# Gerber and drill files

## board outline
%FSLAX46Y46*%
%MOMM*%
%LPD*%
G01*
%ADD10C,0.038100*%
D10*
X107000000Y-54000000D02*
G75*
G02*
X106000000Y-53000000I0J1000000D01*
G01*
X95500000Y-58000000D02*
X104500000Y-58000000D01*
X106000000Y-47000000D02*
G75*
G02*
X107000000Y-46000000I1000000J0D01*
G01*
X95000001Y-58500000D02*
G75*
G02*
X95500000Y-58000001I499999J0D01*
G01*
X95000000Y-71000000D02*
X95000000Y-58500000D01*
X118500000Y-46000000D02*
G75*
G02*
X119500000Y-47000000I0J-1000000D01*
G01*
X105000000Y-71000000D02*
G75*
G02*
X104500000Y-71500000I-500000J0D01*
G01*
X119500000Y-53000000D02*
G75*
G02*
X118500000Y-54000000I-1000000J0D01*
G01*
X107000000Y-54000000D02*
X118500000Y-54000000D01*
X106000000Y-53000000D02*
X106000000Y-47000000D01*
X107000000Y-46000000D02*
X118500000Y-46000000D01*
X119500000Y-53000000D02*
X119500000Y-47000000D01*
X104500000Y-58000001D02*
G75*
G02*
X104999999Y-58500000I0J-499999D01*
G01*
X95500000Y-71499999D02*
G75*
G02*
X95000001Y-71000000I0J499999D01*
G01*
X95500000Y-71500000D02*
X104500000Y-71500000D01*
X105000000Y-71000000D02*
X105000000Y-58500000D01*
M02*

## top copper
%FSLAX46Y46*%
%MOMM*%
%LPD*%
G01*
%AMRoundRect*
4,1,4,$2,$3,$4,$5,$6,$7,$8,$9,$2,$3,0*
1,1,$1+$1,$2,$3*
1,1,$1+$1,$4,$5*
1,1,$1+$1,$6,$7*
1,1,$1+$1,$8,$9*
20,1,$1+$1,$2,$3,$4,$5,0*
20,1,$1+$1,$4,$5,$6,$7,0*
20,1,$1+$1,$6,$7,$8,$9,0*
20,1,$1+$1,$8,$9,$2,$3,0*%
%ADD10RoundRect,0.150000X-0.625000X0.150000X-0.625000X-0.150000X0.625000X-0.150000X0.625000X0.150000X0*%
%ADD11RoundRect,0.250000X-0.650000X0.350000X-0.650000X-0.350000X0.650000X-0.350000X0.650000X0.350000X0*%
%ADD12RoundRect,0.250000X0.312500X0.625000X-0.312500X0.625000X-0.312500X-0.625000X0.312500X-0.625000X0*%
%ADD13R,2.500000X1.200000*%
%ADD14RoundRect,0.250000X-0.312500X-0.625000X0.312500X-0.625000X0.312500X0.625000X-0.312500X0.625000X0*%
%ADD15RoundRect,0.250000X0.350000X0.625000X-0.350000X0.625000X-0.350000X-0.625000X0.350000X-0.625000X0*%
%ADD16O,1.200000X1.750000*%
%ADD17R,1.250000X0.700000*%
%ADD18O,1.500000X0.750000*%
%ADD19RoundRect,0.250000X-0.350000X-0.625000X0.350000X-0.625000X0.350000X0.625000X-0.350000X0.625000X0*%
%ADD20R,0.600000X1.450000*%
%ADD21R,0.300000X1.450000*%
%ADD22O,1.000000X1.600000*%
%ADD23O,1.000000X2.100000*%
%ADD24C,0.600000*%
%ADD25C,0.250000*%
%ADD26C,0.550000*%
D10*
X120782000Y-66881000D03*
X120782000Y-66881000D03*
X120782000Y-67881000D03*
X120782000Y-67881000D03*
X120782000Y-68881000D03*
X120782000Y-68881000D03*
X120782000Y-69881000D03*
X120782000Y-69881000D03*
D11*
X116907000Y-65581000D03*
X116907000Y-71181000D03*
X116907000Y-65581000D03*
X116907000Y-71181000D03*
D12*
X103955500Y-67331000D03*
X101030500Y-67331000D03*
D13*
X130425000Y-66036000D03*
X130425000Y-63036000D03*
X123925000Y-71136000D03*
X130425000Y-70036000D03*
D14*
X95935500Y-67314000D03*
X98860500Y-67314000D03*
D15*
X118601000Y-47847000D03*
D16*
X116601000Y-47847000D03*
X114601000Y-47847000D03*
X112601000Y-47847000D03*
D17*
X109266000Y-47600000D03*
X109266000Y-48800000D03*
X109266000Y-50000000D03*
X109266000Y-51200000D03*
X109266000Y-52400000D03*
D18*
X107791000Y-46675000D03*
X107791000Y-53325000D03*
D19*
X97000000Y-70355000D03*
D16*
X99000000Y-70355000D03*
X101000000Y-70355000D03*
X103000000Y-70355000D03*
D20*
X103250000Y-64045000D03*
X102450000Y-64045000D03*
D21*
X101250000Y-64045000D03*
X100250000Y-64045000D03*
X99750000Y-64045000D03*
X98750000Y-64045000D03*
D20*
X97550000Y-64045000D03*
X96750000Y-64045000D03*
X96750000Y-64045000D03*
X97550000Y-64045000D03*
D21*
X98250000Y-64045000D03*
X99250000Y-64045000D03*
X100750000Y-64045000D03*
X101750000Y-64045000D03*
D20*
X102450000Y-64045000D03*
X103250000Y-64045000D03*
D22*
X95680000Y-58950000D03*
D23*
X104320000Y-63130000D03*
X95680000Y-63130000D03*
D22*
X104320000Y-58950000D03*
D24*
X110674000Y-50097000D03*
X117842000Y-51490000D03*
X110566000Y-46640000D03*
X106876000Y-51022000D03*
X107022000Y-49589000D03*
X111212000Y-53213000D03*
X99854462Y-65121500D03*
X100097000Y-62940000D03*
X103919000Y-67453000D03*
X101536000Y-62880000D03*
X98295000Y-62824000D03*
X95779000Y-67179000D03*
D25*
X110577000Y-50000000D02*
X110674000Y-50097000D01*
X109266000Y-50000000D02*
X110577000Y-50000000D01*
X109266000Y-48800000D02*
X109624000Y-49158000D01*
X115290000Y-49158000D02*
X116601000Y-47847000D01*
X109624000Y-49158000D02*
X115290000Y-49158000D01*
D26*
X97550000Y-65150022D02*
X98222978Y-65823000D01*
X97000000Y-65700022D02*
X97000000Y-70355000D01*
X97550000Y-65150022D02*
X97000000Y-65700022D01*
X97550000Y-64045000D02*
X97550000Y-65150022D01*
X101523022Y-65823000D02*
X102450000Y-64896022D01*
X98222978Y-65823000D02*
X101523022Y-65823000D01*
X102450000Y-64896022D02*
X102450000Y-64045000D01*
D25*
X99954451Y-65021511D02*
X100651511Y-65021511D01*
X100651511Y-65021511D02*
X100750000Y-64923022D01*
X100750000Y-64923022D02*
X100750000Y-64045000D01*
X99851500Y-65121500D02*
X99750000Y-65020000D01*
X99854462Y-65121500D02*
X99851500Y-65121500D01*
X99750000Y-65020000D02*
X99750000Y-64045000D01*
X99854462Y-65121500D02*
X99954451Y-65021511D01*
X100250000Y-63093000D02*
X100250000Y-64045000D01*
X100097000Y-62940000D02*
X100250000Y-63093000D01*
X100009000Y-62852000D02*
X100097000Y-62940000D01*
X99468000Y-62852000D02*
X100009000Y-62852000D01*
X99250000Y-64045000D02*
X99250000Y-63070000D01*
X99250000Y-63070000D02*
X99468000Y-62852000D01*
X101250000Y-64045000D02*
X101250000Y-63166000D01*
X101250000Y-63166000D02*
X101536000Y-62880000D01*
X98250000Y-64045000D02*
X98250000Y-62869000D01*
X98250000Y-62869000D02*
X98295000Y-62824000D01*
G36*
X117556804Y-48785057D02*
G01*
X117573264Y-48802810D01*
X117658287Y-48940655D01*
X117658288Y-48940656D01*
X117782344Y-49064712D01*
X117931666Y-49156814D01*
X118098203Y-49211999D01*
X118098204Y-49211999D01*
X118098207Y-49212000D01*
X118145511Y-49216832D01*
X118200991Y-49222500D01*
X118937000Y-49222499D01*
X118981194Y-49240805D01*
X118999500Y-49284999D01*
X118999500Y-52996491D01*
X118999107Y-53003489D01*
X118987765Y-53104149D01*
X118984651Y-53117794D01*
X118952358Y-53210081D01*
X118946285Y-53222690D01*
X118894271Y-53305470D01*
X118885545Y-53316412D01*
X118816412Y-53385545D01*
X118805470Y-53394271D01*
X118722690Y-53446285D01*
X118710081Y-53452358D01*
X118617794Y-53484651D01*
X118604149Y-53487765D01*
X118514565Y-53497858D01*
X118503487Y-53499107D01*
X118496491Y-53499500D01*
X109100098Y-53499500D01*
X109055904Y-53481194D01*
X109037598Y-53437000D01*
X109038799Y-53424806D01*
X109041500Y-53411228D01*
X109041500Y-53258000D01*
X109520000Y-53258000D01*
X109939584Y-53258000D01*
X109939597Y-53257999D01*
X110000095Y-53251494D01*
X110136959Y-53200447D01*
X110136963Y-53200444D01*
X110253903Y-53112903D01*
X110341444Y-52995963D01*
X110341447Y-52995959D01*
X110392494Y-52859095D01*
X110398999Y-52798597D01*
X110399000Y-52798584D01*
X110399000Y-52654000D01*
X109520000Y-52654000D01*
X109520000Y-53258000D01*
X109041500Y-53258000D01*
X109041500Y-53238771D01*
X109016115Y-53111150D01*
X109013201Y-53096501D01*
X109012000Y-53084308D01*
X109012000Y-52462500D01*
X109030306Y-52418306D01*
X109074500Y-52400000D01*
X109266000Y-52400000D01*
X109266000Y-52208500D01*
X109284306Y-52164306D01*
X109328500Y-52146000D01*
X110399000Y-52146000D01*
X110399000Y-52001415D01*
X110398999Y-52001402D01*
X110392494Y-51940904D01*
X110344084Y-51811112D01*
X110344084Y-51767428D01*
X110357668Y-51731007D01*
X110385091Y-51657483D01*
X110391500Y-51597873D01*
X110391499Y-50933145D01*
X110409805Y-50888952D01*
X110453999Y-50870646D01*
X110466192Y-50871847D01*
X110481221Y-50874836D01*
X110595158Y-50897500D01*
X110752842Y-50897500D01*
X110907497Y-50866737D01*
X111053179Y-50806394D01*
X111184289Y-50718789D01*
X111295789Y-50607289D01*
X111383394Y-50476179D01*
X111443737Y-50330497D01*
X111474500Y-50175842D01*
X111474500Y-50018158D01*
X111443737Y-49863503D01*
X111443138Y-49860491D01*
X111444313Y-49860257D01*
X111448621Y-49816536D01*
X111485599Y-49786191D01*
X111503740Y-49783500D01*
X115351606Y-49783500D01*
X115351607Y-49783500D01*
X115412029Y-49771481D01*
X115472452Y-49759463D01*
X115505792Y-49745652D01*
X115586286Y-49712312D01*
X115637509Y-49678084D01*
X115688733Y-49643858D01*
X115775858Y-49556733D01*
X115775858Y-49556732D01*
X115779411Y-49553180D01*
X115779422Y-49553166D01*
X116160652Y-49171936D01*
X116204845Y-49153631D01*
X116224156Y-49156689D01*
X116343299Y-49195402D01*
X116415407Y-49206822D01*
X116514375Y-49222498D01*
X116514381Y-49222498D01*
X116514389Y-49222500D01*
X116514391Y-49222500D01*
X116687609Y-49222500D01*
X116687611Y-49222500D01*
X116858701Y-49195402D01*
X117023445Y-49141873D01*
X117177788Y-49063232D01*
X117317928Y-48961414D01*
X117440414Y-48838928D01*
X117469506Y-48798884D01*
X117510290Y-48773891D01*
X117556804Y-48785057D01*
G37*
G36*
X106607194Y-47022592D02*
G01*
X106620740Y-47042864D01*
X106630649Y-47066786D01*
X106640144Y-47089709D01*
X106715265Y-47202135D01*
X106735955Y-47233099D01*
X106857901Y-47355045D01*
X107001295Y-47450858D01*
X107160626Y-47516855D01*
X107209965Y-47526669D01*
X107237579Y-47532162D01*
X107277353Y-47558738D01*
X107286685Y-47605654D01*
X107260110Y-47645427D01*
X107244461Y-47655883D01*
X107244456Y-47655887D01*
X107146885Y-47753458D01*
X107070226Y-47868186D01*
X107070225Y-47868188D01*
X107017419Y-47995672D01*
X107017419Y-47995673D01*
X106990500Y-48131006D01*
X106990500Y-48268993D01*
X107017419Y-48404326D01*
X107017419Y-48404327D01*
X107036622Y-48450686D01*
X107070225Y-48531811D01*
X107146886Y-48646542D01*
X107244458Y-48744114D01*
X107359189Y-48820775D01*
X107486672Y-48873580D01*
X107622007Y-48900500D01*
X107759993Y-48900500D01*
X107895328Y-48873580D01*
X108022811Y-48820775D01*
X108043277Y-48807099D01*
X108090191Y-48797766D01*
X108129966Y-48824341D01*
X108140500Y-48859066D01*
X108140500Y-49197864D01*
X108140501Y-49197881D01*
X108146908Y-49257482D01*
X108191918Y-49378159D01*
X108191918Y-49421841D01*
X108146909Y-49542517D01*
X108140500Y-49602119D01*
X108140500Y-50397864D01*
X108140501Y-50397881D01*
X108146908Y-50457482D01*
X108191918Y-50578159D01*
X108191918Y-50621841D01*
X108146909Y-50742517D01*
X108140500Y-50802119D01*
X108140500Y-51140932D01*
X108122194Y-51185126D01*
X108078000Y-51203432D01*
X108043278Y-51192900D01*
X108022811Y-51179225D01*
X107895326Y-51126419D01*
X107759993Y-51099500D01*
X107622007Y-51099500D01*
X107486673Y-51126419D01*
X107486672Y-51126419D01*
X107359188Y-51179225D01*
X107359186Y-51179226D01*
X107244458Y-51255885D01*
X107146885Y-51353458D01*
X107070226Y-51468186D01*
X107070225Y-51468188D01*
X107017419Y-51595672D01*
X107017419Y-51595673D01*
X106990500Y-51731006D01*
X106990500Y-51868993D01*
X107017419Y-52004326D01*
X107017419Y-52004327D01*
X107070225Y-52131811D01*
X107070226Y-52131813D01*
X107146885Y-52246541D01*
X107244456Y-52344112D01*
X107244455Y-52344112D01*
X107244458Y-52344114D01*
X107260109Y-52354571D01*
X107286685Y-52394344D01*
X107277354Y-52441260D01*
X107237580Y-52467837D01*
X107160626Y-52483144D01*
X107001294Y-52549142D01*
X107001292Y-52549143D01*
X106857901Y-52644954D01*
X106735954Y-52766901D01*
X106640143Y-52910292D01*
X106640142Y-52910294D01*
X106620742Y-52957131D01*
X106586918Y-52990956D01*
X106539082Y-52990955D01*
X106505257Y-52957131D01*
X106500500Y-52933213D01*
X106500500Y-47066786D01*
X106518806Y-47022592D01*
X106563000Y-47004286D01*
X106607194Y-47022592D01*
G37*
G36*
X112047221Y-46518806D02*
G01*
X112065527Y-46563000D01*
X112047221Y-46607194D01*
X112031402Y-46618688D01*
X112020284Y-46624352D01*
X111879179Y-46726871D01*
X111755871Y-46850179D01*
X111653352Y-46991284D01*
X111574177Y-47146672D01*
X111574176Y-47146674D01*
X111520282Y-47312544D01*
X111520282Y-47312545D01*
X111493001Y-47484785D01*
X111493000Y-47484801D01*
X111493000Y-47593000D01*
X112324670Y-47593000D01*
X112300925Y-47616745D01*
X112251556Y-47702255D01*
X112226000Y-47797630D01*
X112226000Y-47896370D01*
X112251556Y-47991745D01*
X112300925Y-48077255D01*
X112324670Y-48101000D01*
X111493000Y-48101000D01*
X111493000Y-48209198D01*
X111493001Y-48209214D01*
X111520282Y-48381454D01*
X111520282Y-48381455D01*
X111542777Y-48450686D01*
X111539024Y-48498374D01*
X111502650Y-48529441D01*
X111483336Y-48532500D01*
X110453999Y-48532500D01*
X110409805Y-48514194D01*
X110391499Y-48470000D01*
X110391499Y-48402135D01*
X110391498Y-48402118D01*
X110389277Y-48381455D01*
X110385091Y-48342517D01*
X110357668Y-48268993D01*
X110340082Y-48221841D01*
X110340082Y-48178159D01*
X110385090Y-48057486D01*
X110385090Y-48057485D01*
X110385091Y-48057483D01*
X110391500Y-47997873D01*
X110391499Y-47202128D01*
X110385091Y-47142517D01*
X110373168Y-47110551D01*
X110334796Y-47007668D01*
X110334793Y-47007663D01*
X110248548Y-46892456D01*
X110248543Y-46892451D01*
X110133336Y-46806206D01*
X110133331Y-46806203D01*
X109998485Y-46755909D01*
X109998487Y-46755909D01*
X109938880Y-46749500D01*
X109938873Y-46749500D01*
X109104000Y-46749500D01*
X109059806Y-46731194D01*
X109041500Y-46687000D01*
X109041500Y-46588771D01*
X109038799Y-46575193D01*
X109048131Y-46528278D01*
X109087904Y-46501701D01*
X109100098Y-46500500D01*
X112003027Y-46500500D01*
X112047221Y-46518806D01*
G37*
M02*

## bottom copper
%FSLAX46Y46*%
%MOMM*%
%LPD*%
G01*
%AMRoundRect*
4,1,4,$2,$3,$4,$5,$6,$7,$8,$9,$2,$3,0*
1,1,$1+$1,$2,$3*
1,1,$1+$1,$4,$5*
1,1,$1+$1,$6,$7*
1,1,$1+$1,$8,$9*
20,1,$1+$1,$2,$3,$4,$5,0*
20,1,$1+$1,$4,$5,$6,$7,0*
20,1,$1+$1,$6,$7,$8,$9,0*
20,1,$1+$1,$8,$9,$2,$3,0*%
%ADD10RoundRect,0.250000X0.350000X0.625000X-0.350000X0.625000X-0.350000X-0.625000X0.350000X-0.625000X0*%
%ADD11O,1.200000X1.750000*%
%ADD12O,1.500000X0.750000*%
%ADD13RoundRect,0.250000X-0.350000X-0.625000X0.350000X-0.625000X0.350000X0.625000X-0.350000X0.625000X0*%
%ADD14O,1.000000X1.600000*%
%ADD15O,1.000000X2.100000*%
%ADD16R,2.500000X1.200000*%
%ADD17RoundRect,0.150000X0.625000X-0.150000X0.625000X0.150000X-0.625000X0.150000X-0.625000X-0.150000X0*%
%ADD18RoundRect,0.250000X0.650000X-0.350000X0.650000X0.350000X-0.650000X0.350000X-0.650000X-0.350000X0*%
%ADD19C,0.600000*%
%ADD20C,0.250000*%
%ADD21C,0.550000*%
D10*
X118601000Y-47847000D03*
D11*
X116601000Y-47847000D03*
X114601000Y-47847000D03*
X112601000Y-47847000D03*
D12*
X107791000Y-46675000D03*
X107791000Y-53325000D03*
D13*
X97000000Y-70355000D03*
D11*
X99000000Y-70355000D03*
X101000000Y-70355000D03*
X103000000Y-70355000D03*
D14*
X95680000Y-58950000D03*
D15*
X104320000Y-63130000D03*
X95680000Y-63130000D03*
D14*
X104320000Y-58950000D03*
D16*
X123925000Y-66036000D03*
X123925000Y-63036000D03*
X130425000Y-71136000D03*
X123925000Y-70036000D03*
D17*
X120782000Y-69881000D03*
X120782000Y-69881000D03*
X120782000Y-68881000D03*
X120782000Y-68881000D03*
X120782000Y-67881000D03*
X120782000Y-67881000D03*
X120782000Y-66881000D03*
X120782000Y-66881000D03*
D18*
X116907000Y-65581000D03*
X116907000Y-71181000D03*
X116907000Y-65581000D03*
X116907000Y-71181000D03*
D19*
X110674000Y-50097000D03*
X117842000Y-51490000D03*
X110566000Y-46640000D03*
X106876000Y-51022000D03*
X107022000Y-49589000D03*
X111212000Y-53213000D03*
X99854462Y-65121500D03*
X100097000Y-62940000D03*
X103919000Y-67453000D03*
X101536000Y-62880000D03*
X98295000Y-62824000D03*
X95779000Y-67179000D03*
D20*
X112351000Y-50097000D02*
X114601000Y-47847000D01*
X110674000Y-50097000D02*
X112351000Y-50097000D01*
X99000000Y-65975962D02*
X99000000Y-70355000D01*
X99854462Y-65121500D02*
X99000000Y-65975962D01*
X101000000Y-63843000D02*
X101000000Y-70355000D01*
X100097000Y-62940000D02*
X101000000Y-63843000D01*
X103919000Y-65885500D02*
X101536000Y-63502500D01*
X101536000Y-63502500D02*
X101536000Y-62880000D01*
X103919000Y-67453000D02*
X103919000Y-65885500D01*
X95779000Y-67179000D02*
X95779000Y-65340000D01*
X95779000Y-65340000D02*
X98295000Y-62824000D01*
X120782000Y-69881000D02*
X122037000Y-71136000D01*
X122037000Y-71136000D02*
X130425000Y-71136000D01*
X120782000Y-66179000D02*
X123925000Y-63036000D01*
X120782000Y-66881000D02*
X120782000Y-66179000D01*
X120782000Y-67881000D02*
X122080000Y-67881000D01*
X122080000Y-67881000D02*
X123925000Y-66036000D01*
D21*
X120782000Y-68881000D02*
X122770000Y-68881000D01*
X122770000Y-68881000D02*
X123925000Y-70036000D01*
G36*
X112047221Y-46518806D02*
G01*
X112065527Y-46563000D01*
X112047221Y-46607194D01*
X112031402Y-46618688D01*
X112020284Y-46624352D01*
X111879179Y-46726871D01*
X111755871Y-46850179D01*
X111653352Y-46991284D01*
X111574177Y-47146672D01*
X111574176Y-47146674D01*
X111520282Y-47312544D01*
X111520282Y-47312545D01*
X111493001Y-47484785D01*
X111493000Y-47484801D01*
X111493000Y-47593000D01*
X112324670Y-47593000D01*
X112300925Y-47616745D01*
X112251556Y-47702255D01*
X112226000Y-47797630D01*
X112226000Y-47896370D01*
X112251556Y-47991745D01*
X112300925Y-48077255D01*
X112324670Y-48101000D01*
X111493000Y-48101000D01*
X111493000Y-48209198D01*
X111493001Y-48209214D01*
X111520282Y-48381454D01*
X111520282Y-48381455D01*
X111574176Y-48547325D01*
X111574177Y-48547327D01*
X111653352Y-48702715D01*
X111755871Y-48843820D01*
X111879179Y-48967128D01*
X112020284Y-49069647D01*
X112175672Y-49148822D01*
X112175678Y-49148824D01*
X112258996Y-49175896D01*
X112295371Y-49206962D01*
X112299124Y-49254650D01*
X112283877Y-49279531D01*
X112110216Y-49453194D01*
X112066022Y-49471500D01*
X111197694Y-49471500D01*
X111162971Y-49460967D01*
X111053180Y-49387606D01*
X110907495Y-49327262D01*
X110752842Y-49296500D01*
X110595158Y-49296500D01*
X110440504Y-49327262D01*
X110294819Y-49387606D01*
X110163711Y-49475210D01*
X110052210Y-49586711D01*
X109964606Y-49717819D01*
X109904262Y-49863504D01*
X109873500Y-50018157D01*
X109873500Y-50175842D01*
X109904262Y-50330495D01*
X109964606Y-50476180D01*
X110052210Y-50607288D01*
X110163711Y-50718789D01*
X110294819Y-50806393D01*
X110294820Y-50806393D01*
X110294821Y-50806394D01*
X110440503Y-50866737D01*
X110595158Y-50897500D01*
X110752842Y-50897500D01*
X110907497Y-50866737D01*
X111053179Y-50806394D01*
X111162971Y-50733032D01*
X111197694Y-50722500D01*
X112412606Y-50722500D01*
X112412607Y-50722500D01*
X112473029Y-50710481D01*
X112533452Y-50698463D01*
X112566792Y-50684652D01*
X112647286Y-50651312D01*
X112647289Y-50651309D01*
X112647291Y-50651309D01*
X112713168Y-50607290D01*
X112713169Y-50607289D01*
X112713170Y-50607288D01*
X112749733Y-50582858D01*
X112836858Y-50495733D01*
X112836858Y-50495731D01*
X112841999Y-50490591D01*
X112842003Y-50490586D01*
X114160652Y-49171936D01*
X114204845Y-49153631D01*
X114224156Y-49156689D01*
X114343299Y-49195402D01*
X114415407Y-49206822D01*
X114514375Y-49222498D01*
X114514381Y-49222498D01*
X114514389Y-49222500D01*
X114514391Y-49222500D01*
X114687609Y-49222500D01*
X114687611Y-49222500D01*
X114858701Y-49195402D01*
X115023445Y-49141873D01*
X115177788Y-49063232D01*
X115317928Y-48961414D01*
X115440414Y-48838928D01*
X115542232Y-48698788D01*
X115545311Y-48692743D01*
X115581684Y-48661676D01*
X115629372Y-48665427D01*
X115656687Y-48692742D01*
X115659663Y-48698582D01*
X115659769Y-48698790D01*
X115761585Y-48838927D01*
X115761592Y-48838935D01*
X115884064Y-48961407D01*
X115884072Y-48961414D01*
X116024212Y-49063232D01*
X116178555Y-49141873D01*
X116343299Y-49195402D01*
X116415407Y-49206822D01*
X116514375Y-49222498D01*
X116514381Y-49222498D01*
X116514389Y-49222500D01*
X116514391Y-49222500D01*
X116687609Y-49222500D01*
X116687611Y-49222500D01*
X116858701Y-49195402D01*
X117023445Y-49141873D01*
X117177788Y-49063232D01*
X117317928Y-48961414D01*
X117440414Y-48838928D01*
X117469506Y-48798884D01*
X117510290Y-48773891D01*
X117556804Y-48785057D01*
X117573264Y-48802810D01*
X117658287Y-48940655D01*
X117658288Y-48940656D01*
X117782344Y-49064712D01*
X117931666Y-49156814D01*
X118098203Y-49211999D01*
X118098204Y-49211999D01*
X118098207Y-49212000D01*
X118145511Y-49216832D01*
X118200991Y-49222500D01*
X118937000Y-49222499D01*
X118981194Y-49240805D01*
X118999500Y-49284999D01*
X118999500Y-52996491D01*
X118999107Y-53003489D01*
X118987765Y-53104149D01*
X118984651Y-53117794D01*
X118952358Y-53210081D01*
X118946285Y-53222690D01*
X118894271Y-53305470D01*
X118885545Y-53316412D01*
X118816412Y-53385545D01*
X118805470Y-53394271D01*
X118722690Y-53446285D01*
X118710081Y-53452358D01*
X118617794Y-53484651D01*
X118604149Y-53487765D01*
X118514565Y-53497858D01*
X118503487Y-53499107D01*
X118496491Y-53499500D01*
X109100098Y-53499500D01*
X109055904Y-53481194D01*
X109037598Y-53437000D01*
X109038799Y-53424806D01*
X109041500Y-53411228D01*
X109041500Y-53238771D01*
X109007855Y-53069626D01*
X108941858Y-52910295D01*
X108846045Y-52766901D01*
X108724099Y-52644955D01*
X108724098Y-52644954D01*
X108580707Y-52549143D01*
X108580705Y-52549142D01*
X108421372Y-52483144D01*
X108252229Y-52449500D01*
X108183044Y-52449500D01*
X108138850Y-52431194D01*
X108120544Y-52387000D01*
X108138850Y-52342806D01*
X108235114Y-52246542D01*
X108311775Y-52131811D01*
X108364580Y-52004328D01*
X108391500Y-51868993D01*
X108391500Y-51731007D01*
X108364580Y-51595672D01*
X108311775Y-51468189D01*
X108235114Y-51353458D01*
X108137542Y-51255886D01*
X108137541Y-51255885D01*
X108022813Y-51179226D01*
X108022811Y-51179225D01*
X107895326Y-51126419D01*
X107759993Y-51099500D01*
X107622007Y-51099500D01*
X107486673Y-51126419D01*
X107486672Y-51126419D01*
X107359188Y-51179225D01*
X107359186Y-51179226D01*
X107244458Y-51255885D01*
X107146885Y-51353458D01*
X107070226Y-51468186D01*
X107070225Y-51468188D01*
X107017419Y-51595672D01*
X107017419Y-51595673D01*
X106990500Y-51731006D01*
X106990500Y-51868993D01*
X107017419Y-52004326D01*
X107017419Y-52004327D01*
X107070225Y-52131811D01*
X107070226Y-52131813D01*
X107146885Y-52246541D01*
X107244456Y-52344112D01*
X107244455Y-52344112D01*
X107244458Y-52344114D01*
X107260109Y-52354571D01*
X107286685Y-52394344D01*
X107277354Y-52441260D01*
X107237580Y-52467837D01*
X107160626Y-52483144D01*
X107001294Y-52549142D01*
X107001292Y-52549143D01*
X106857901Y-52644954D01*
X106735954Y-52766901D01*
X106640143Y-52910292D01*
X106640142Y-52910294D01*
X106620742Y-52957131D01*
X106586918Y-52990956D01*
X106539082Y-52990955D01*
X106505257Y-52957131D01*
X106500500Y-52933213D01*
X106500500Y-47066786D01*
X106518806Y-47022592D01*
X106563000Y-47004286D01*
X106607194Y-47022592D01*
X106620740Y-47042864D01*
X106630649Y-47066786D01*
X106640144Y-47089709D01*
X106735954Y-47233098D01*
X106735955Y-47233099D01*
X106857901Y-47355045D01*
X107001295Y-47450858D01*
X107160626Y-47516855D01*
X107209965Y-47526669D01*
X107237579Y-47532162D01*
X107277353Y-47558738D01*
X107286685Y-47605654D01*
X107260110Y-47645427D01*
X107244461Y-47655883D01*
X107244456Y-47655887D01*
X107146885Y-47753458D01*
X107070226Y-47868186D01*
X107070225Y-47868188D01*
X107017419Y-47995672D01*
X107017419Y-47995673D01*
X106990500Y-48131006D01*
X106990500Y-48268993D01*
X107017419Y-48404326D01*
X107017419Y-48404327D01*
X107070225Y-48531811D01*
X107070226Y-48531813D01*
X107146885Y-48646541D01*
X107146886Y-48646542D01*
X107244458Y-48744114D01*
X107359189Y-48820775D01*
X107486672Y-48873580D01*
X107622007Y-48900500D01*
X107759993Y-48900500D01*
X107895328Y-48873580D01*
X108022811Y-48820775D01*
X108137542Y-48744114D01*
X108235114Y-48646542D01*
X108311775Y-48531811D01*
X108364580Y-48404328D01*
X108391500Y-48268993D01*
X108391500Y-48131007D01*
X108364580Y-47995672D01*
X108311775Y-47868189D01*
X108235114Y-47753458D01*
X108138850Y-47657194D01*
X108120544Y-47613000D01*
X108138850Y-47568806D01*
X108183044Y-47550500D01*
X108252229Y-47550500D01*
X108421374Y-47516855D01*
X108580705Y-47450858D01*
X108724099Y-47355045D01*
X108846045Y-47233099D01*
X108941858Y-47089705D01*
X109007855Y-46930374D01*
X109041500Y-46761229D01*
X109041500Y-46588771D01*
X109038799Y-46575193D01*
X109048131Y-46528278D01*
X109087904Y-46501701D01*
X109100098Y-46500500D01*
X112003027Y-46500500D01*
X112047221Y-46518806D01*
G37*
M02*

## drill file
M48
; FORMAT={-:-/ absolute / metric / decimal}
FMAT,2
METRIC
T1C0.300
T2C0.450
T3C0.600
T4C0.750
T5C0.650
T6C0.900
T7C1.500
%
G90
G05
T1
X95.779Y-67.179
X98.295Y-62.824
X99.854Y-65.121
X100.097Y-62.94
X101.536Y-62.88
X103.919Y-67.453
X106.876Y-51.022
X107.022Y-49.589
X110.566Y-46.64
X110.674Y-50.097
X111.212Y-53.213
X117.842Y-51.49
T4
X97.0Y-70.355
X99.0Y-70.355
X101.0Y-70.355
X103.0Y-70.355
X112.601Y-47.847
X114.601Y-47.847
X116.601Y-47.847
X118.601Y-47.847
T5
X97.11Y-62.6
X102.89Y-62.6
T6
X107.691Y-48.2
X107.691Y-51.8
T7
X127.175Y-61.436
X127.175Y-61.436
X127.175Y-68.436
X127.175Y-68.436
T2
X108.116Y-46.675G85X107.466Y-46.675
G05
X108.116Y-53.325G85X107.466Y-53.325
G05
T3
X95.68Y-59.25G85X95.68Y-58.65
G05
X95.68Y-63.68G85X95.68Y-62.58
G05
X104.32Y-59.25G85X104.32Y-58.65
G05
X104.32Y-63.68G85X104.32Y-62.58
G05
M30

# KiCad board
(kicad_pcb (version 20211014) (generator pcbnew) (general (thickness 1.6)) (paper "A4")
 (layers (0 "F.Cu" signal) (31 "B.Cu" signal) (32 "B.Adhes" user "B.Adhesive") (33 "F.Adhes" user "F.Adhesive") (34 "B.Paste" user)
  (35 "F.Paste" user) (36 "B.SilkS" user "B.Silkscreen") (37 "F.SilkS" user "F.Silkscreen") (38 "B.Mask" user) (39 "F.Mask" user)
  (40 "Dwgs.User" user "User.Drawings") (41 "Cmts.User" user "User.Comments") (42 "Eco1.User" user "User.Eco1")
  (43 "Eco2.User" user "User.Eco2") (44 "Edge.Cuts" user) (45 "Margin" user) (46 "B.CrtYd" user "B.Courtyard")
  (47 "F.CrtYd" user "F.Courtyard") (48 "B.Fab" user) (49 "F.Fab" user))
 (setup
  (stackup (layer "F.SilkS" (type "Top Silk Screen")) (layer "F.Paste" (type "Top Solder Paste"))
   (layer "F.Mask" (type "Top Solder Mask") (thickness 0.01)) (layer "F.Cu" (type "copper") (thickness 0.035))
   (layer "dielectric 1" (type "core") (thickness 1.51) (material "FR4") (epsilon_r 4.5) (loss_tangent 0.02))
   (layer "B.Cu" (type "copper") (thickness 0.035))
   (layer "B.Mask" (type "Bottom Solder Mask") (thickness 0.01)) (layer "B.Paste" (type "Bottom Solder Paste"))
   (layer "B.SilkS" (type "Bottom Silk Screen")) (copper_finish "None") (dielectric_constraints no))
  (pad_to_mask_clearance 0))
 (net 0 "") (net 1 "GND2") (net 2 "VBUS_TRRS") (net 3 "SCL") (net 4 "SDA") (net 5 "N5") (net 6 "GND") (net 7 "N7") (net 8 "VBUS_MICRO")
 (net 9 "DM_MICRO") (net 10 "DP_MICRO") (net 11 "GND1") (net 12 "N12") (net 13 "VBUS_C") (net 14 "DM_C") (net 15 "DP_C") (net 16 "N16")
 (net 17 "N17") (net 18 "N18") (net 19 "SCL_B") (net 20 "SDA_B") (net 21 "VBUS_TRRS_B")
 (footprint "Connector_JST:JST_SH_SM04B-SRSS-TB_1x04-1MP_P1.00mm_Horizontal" (layer "F.Cu") (at 118.782 68.381 -90)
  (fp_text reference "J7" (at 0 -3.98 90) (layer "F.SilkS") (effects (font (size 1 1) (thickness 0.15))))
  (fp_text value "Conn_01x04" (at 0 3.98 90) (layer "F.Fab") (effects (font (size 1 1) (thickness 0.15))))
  (pad "1" smd roundrect (at -1.5 -2 270) (size 0.6 1.55) (layers "F.Cu" "F.Paste" "F.Mask") (roundrect_rratio 0.25) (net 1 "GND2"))
  (pad "1" smd roundrect (at -1.5 -2 270) (size 0.6 1.55) (layers "F.Cu" "F.Paste" "F.Mask") (roundrect_rratio 0.25) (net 1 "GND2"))
  (pad "2" smd roundrect (at -0.5 -2 270) (size 0.6 1.55) (layers "F.Cu" "F.Paste" "F.Mask") (roundrect_rratio 0.25) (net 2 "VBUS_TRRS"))
  (pad "2" smd roundrect (at -0.5 -2 270) (size 0.6 1.55) (layers "F.Cu" "F.Paste" "F.Mask") (roundrect_rratio 0.25) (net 2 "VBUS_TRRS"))
  (pad "3" smd roundrect (at 0.5 -2 270) (size 0.6 1.55) (layers "F.Cu" "F.Paste" "F.Mask") (roundrect_rratio 0.25) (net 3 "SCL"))
  (pad "3" smd roundrect (at 0.5 -2 270) (size 0.6 1.55) (layers "F.Cu" "F.Paste" "F.Mask") (roundrect_rratio 0.25) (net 3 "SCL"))
  (pad "4" smd roundrect (at 1.5 -2 270) (size 0.6 1.55) (layers "F.Cu" "F.Paste" "F.Mask") (roundrect_rratio 0.25) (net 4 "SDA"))
  (pad "4" smd roundrect (at 1.5 -2 270) (size 0.6 1.55) (layers "F.Cu" "F.Paste" "F.Mask") (roundrect_rratio 0.25) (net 4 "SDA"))
  (pad "MP" smd roundrect (at -2.8 1.875 270) (size 1.2 1.8) (layers "F.Cu" "F.Paste" "F.Mask") (roundrect_rratio 0.208333))
  (pad "MP" smd roundrect (at 2.8 1.875 270) (size 1.2 1.8) (layers "F.Cu" "F.Paste" "F.Mask") (roundrect_rratio 0.208333))
  (pad "MP" smd roundrect (at -2.8 1.875 270) (size 1.2 1.8) (layers "F.Cu" "F.Paste" "F.Mask") (roundrect_rratio 0.208333))
  (pad "MP" smd roundrect (at 2.8 1.875 270) (size 1.2 1.8) (layers "F.Cu" "F.Paste" "F.Mask") (roundrect_rratio 0.208333)))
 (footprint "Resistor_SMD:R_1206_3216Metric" (layer "F.Cu") (at 102.493 67.331 180)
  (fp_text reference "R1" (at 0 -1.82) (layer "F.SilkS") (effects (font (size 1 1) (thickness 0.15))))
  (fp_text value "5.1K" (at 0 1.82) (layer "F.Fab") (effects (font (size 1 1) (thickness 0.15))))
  (pad "1" smd roundrect (at -1.4625 0 180) (size 1.125 1.75) (layers "F.Cu" "F.Paste" "F.Mask") (roundrect_rratio 0.222222) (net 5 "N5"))
  (pad "2" smd roundrect (at 1.4625 0 180) (size 1.125 1.75) (layers "F.Cu" "F.Paste" "F.Mask") (roundrect_rratio 0.222222) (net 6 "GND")))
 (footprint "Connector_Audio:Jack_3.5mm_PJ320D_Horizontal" (layer "F.Cu") (at 127.175 66.211 -90)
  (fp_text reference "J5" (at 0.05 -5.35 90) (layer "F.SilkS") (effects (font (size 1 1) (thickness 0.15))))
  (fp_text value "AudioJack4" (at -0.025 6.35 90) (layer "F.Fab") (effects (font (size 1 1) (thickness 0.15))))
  (pad "" np_thru_hole circle (at -4.775 0 270) (size 1.5 1.5) (drill 1.5) (layers *.Cu *.Mask))
  (pad "" np_thru_hole circle (at 2.225 0 270) (size 1.5 1.5) (drill 1.5) (layers *.Cu *.Mask))
  (pad "R1" smd rect (at -0.175 -3.25 270) (size 1.2 2.5) (layers "F.Cu" "F.Paste" "F.Mask") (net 3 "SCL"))
  (pad "R2" smd rect (at -3.175 -3.25 270) (size 1.2 2.5) (layers "F.Cu" "F.Paste" "F.Mask") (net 4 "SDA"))
  (pad "S" smd rect (at 4.925 3.25 270) (size 1.2 2.5) (layers "F.Cu" "F.Paste" "F.Mask") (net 1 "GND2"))
  (pad "T" smd rect (at 3.825 -3.25 270) (size 1.2 2.5) (layers "F.Cu" "F.Paste" "F.Mask") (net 2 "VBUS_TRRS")))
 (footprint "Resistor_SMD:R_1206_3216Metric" (layer "F.Cu") (at 97.398 67.314)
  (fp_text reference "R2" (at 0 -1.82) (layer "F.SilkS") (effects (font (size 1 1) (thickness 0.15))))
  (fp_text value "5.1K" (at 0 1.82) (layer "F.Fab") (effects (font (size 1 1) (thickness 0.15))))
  (pad "1" smd roundrect (at -1.4625 0) (size 1.125 1.75) (layers "F.Cu" "F.Paste" "F.Mask") (roundrect_rratio 0.222222) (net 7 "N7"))
  (pad "2" smd roundrect (at 1.4625 0) (size 1.125 1.75) (layers "F.Cu" "F.Paste" "F.Mask") (roundrect_rratio 0.222222) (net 6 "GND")))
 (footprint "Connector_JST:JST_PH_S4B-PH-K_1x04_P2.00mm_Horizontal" (layer "F.Cu") (at 118.601 47.847 180)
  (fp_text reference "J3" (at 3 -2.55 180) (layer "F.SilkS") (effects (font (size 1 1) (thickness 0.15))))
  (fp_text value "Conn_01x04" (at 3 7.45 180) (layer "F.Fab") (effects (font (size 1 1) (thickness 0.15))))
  (pad "1" thru_hole roundrect (at 0 0 180) (size 1.2 1.75) (drill 0.75) (layers *.Cu *.Mask) (roundrect_rratio 0.208333)
   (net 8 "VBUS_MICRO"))
  (pad "2" thru_hole oval (at 2 0 180) (size 1.2 1.75) (drill 0.75) (layers *.Cu *.Mask) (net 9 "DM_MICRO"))
  (pad "3" thru_hole oval (at 4 0 180) (size 1.2 1.75) (drill 0.75) (layers *.Cu *.Mask) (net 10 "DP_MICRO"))
  (pad "4" thru_hole oval (at 6 0 180) (size 1.2 1.75) (drill 0.75) (layers *.Cu *.Mask) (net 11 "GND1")))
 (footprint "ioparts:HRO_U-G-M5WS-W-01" (layer "F.Cu") (at 107.691 50 -90)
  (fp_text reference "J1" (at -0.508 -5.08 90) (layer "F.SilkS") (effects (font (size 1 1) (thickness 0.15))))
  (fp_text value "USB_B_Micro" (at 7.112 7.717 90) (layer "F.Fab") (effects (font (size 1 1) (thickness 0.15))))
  (pad "" np_thru_hole circle locked (at 1.8 0 270) (size 0.9 0.9) (drill 0.9) (layers *.Cu *.Mask))
  (pad "" np_thru_hole circle locked (at -1.8 0 270) (size 0.9 0.9) (drill 0.9) (layers *.Cu *.Mask))
  (pad "1" smd rect locked (at -2.4 -1.575 270) (size 0.7 1.25) (layers "F.Cu" "F.Paste" "F.Mask") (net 8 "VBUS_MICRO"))
  (pad "2" smd rect locked (at -1.2 -1.575 270) (size 0.7 1.25) (layers "F.Cu" "F.Paste" "F.Mask") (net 9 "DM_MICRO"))
  (pad "3" smd rect locked (at 0 -1.575 270) (size 0.7 1.25) (layers "F.Cu" "F.Paste" "F.Mask") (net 10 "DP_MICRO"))
  (pad "4" smd rect locked (at 1.2 -1.575 270) (size 0.7 1.25) (layers "F.Cu" "F.Paste" "F.Mask") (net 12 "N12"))
  (pad "5" smd rect locked (at 2.4 -1.575 270) (size 0.7 1.25) (layers "F.Cu" "F.Paste" "F.Mask") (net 11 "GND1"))
  (pad "S1" thru_hole oval locked (at -3.325 -0.1 270) (size 0.75 1.5) (drill oval 0.45 1.1) (layers *.Cu *.Mask))
  (pad "S2" thru_hole oval locked (at 3.325 -0.1 270) (size 0.75 1.5) (drill oval 0.45 1.1) (layers *.Cu *.Mask)))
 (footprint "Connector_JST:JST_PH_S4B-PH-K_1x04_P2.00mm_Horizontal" (layer "F.Cu") (at 97 70.355)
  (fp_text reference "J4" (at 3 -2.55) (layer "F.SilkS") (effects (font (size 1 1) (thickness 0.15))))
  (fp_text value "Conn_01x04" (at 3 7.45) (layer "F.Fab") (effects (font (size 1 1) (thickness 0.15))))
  (pad "1" thru_hole roundrect (at 0 0) (size 1.2 1.75) (drill 0.75) (layers *.Cu *.Mask) (roundrect_rratio 0.208333) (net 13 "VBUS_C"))
  (pad "2" thru_hole oval (at 2 0) (size 1.2 1.75) (drill 0.75) (layers *.Cu *.Mask) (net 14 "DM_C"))
  (pad "3" thru_hole oval (at 4 0) (size 1.2 1.75) (drill 0.75) (layers *.Cu *.Mask) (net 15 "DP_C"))
  (pad "4" thru_hole oval (at 6 0) (size 1.2 1.75) (drill 0.75) (layers *.Cu *.Mask) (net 6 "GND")))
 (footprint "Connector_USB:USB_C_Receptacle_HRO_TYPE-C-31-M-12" (layer "F.Cu") (at 100 60 180)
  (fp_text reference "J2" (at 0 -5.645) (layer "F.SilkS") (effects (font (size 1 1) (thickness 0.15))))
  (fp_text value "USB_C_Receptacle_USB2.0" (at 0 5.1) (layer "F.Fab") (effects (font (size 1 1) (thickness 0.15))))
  (pad "" np_thru_hole circle (at -2.89 -2.6 180) (size 0.65 0.65) (drill 0.65) (layers *.Cu *.Mask))
  (pad "" np_thru_hole circle (at 2.89 -2.6 180) (size 0.65 0.65) (drill 0.65) (layers *.Cu *.Mask))
  (pad "A1" smd rect (at -3.25 -4.045 180) (size 0.6 1.45) (layers "F.Cu" "F.Paste" "F.Mask") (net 6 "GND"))
  (pad "A4" smd rect (at -2.45 -4.045 180) (size 0.6 1.45) (layers "F.Cu" "F.Paste" "F.Mask") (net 13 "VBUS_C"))
  (pad "A5" smd rect (at -1.25 -4.045 180) (size 0.3 1.45) (layers "F.Cu" "F.Paste" "F.Mask") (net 5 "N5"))
  (pad "A6" smd rect (at -0.25 -4.045 180) (size 0.3 1.45) (layers "F.Cu" "F.Paste" "F.Mask") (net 15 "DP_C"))
  (pad "A7" smd rect (at 0.25 -4.045 180) (size 0.3 1.45) (layers "F.Cu" "F.Paste" "F.Mask") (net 14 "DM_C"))
  (pad "A8" smd rect (at 1.25 -4.045 180) (size 0.3 1.45) (layers "F.Cu" "F.Paste" "F.Mask") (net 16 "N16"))
  (pad "A9" smd rect (at 2.45 -4.045 180) (size 0.6 1.45) (layers "F.Cu" "F.Paste" "F.Mask") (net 13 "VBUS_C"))
  (pad "A12" smd rect (at 3.25 -4.045 180) (size 0.6 1.45) (layers "F.Cu" "F.Paste" "F.Mask") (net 6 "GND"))
  (pad "B1" smd rect (at 3.25 -4.045 180) (size 0.6 1.45) (layers "F.Cu" "F.Paste" "F.Mask") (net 6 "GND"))
  (pad "B4" smd rect (at 2.45 -4.045 180) (size 0.6 1.45) (layers "F.Cu" "F.Paste" "F.Mask") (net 13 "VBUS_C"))
  (pad "B5" smd rect (at 1.75 -4.045 180) (size 0.3 1.45) (layers "F.Cu" "F.Paste" "F.Mask") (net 7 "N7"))
  (pad "B6" smd rect (at 0.75 -4.045 180) (size 0.3 1.45) (layers "F.Cu" "F.Paste" "F.Mask") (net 15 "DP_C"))
  (pad "B7" smd rect (at -0.75 -4.045 180) (size 0.3 1.45) (layers "F.Cu" "F.Paste" "F.Mask") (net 14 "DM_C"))
  (pad "B8" smd rect (at -1.75 -4.045 180) (size 0.3 1.45) (layers "F.Cu" "F.Paste" "F.Mask") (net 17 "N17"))
  (pad "B9" smd rect (at -2.45 -4.045 180) (size 0.6 1.45) (layers "F.Cu" "F.Paste" "F.Mask") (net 13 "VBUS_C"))
  (pad "B12" smd rect (at -3.25 -4.045 180) (size 0.6 1.45) (layers "F.Cu" "F.Paste" "F.Mask") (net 6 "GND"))
  (pad "S1" thru_hole oval (at 4.32 1.05 180) (size 1 1.6) (drill oval 0.6 1.2) (layers *.Cu *.Mask) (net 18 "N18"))
  (pad "S1" thru_hole oval (at -4.32 -3.13 180) (size 1 2.1) (drill oval 0.6 1.7) (layers *.Cu *.Mask) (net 18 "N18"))
  (pad "S1" thru_hole oval (at 4.32 -3.13 180) (size 1 2.1) (drill oval 0.6 1.7) (layers *.Cu *.Mask) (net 18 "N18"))
  (pad "S1" thru_hole oval (at -4.32 1.05 180) (size 1 1.6) (drill oval 0.6 1.2) (layers *.Cu *.Mask) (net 18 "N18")))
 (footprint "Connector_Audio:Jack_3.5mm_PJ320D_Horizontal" (layer "B.Cu") (at 127.175 66.211 -90)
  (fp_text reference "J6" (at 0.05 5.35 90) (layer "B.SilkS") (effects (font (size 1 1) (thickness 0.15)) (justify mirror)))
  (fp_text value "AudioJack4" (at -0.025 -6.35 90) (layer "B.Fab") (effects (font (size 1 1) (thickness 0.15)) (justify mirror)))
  (pad "" np_thru_hole circle (at -4.775 0 270) (size 1.5 1.5) (drill 1.5) (layers *.Cu *.Mask))
  (pad "" np_thru_hole circle (at 2.225 0 270) (size 1.5 1.5) (drill 1.5) (layers *.Cu *.Mask))
  (pad "R1" smd rect (at -0.175 3.25 270) (size 1.2 2.5) (layers "B.Cu" "B.Paste" "B.Mask") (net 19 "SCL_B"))
  (pad "R2" smd rect (at -3.175 3.25 270) (size 1.2 2.5) (layers "B.Cu" "B.Paste" "B.Mask") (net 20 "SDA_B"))
  (pad "S" smd rect (at 4.925 -3.25 270) (size 1.2 2.5) (layers "B.Cu" "B.Paste" "B.Mask") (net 1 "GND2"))
  (pad "T" smd rect (at 3.825 3.25 270) (size 1.2 2.5) (layers "B.Cu" "B.Paste" "B.Mask") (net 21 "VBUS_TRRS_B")))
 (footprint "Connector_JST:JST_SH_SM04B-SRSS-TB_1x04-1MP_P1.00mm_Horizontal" (layer "B.Cu") (at 118.782 68.381 90)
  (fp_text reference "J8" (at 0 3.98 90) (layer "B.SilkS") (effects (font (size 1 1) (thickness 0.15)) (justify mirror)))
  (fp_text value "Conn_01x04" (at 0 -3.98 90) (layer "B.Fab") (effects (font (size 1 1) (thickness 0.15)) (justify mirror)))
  (pad "1" smd roundrect (at -1.5 2 90) (size 0.6 1.55) (layers "B.Cu" "B.Paste" "B.Mask") (roundrect_rratio 0.25) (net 1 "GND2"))
  (pad "1" smd roundrect (at -1.5 2 90) (size 0.6 1.55) (layers "B.Cu" "B.Paste" "B.Mask") (roundrect_rratio 0.25) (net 1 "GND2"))
  (pad "2" smd roundrect (at -0.5 2 90) (size 0.6 1.55) (layers "B.Cu" "B.Paste" "B.Mask") (roundrect_rratio 0.25) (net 21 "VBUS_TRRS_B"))
  (pad "2" smd roundrect (at -0.5 2 90) (size 0.6 1.55) (layers "B.Cu" "B.Paste" "B.Mask") (roundrect_rratio 0.25) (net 21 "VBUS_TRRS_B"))
  (pad "3" smd roundrect (at 0.5 2 90) (size 0.6 1.55) (layers "B.Cu" "B.Paste" "B.Mask") (roundrect_rratio 0.25) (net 19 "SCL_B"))
  (pad "3" smd roundrect (at 0.5 2 90) (size 0.6 1.55) (layers "B.Cu" "B.Paste" "B.Mask") (roundrect_rratio 0.25) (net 19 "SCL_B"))
  (pad "4" smd roundrect (at 1.5 2 90) (size 0.6 1.55) (layers "B.Cu" "B.Paste" "B.Mask") (roundrect_rratio 0.25) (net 20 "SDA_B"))
  (pad "4" smd roundrect (at 1.5 2 90) (size 0.6 1.55) (layers "B.Cu" "B.Paste" "B.Mask") (roundrect_rratio 0.25) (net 20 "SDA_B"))
  (pad "MP" smd roundrect (at 2.8 -1.875 90) (size 1.2 1.8) (layers "B.Cu" "B.Paste" "B.Mask") (roundrect_rratio 0.208333))
  (pad "MP" smd roundrect (at -2.8 -1.875 90) (size 1.2 1.8) (layers "B.Cu" "B.Paste" "B.Mask") (roundrect_rratio 0.208333))
  (pad "MP" smd roundrect (at 2.8 -1.875 90) (size 1.2 1.8) (layers "B.Cu" "B.Paste" "B.Mask") (roundrect_rratio 0.208333))
  (pad "MP" smd roundrect (at -2.8 -1.875 90) (size 1.2 1.8) (layers "B.Cu" "B.Paste" "B.Mask") (roundrect_rratio 0.208333)))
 (gr_arc (start 107 54) (mid 106.292893 53.707107) (end 106 53) (layer "Edge.Cuts") (width 0.0381))
 (gr_line (start 95.5 58) (end 104.5 58) (layer "Edge.Cuts") (width 0.0381))
 (gr_arc (start 106 47) (mid 106.292893 46.292893) (end 107 46) (layer "Edge.Cuts") (width 0.0381))
 (gr_arc (start 95.000001 58.5) (mid 95.146447 58.146447) (end 95.5 58.000001) (layer "Edge.Cuts") (width 0.0381))
 (gr_line (start 95 71) (end 95 58.5) (layer "Edge.Cuts") (width 0.0381))
 (gr_arc (start 118.5 46) (mid 119.207107 46.292893) (end 119.5 47) (layer "Edge.Cuts") (width 0.0381))
 (gr_arc (start 105 71) (mid 104.853553 71.353553) (end 104.5 71.5) (layer "Edge.Cuts") (width 0.0381))
 (gr_arc (start 119.5 53) (mid 119.207107 53.707107) (end 118.5 54) (layer "Edge.Cuts") (width 0.0381))
 (gr_line (start 107 54) (end 118.5 54) (layer "Edge.Cuts") (width 0.0381))
 (gr_line (start 106 53) (end 106 47) (layer "Edge.Cuts") (width 0.0381))
 (gr_line (start 107 46) (end 118.5 46) (layer "Edge.Cuts") (width 0.0381))
 (gr_line (start 119.5 53) (end 119.5 47) (layer "Edge.Cuts") (width 0.0381))
 (gr_arc (start 104.5 58.000001) (mid 104.853553 58.146447) (end 104.999999 58.5) (layer "Edge.Cuts") (width 0.0381))
 (gr_arc (start 95.5 71.499999) (mid 95.146447 71.353553) (end 95.000001 71) (layer "Edge.Cuts") (width 0.0381))
 (gr_line (start 95.5 71.5) (end 104.5 71.5) (layer "Edge.Cuts") (width 0.0381))
 (gr_line (start 105 71) (end 105 58.5) (layer "Edge.Cuts") (width 0.0381))
 (segment (start 110.577 50) (end 110.674 50.097) (width 0.25) (layer "F.Cu") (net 10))
 (segment (start 109.266 50) (end 110.577 50) (width 0.25) (layer "F.Cu") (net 10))
 (via (at 110.674 50.097) (size 0.6) (drill 0.3) (layers "F.Cu" "B.Cu") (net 10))
 (segment (start 112.351 50.097) (end 114.601 47.847) (width 0.25) (layer "B.Cu") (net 10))
 (segment (start 110.674 50.097) (end 112.351 50.097) (width 0.25) (layer "B.Cu") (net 10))
 (segment (start 109.266 48.8) (end 109.624 49.158) (width 0.25) (layer "F.Cu") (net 9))
 (segment (start 115.29 49.158) (end 116.601 47.847) (width 0.25) (layer "F.Cu") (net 9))
 (segment (start 109.624 49.158) (end 115.29 49.158) (width 0.25) (layer "F.Cu") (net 9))
 (via (at 117.842 51.49) (size 0.6) (drill 0.3) (layers "F.Cu" "B.Cu") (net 11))
 (via (at 110.566 46.64) (size 0.6) (drill 0.3) (layers "F.Cu" "B.Cu") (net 11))
 (via (at 106.876 51.022) (size 0.6) (drill 0.3) (layers "F.Cu" "B.Cu") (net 11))
 (via (at 107.022 49.589) (size 0.6) (drill 0.3) (layers "F.Cu" "B.Cu") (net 11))
 (via (at 111.212 53.213) (size 0.6) (drill 0.3) (layers "F.Cu" "B.Cu") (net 11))
 (segment (start 97.55 65.150022) (end 98.222978 65.823) (width 0.55) (layer "F.Cu") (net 13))
 (segment (start 97 65.700022) (end 97 70.355) (width 0.55) (layer "F.Cu") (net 13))
 (segment (start 97.55 65.150022) (end 97 65.700022) (width 0.55) (layer "F.Cu") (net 13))
 (segment (start 97.55 64.045) (end 97.55 65.150022) (width 0.55) (layer "F.Cu") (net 13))
 (segment (start 101.523022 65.823) (end 102.45 64.896022) (width 0.55) (layer "F.Cu") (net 13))
 (segment (start 98.222978 65.823) (end 101.523022 65.823) (width 0.55) (layer "F.Cu") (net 13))
 (segment (start 102.45 64.896022) (end 102.45 64.045) (width 0.55) (layer "F.Cu") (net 13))
 (segment (start 99.954451 65.021511) (end 100.651511 65.021511) (width 0.25) (layer "F.Cu") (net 14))
 (segment (start 100.651511 65.021511) (end 100.75 64.923022) (width 0.25) (layer "F.Cu") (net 14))
 (segment (start 100.75 64.923022) (end 100.75 64.045) (width 0.25) (layer "F.Cu") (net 14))
 (segment (start 99.8515 65.1215) (end 99.75 65.02) (width 0.25) (layer "F.Cu") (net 14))
 (segment (start 99.854462 65.1215) (end 99.8515 65.1215) (width 0.25) (layer "F.Cu") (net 14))
 (segment (start 99.75 65.02) (end 99.75 64.045) (width 0.25) (layer "F.Cu") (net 14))
 (segment (start 99.854462 65.1215) (end 99.954451 65.021511) (width 0.25) (layer "F.Cu") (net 14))
 (via (at 99.854462 65.1215) (size 0.6) (drill 0.3) (layers "F.Cu" "B.Cu") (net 14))
 (segment (start 99 65.975962) (end 99 70.355) (width 0.25) (layer "B.Cu") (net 14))
 (segment (start 99.854462 65.1215) (end 99 65.975962) (width 0.25) (layer "B.Cu") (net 14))
 (segment (start 100.25 63.093) (end 100.25 64.045) (width 0.25) (layer "F.Cu") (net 15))
 (segment (start 100.097 62.94) (end 100.25 63.093) (width 0.25) (layer "F.Cu") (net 15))
 (segment (start 100.009 62.852) (end 100.097 62.94) (width 0.25) (layer "F.Cu") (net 15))
 (segment (start 99.468 62.852) (end 100.009 62.852) (width 0.25) (layer "F.Cu") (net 15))
 (segment (start 99.25 64.045) (end 99.25 63.07) (width 0.25) (layer "F.Cu") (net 15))
 (segment (start 99.25 63.07) (end 99.468 62.852) (width 0.25) (layer "F.Cu") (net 15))
 (via (at 100.097 62.94) (size 0.6) (drill 0.3) (layers "F.Cu" "B.Cu") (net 15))
 (segment (start 101 63.843) (end 101 70.355) (width 0.25) (layer "B.Cu") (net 15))
 (segment (start 100.097 62.94) (end 101 63.843) (width 0.25) (layer "B.Cu") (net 15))
 (segment (start 101.25 64.045) (end 101.25 63.166) (width 0.25) (layer "F.Cu") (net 5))
 (segment (start 101.25 63.166) (end 101.536 62.88) (width 0.25) (layer "F.Cu") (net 5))
 (via (at 103.919 67.453) (size 0.6) (drill 0.3) (layers "F.Cu" "B.Cu") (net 5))
 (via (at 101.536 62.88) (size 0.6) (drill 0.3) (layers "F.Cu" "B.Cu") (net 5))
 (segment (start 103.919 65.8855) (end 101.536 63.5025) (width 0.25) (layer "B.Cu") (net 5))
 (segment (start 101.536 63.5025) (end 101.536 62.88) (width 0.25) (layer "B.Cu") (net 5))
 (segment (start 103.919 67.453) (end 103.919 65.8855) (width 0.25) (layer "B.Cu") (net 5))
 (segment (start 98.25 64.045) (end 98.25 62.869) (width 0.25) (layer "F.Cu") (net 7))
 (segment (start 98.25 62.869) (end 98.295 62.824) (width 0.25) (layer "F.Cu") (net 7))
 (via (at 98.295 62.824) (size 0.6) (drill 0.3) (layers "F.Cu" "B.Cu") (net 7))
 (via (at 95.779 67.179) (size 0.6) (drill 0.3) (layers "F.Cu" "B.Cu") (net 7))
 (segment (start 95.779 67.179) (end 95.779 65.34) (width 0.25) (layer "B.Cu") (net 7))
 (segment (start 95.779 65.34) (end 98.295 62.824) (width 0.25) (layer "B.Cu") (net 7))
 (segment (start 120.782 69.881) (end 122.037 71.136) (width 0.25) (layer "B.Cu") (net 1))
 (segment (start 122.037 71.136) (end 130.425 71.136) (width 0.25) (layer "B.Cu") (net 1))
 (segment (start 120.782 66.179) (end 123.925 63.036) (width 0.25) (layer "B.Cu") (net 20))
 (segment (start 120.782 66.881) (end 120.782 66.179) (width 0.25) (layer "B.Cu") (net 20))
 (segment (start 120.782 67.881) (end 122.08 67.881) (width 0.25) (layer "B.Cu") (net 19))
 (segment (start 122.08 67.881) (end 123.925 66.036) (width 0.25) (layer "B.Cu") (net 19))
 (segment (start 120.782 68.881) (end 122.77 68.881) (width 0.55) (layer "B.Cu") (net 21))
 (segment (start 122.77 68.881) (end 123.925 70.036) (width 0.55) (layer "B.Cu") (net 21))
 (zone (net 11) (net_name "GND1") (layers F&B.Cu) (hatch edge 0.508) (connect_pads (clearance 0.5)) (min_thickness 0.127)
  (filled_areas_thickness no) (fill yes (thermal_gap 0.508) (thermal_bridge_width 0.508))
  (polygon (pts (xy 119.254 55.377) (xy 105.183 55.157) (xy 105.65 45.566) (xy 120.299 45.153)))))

